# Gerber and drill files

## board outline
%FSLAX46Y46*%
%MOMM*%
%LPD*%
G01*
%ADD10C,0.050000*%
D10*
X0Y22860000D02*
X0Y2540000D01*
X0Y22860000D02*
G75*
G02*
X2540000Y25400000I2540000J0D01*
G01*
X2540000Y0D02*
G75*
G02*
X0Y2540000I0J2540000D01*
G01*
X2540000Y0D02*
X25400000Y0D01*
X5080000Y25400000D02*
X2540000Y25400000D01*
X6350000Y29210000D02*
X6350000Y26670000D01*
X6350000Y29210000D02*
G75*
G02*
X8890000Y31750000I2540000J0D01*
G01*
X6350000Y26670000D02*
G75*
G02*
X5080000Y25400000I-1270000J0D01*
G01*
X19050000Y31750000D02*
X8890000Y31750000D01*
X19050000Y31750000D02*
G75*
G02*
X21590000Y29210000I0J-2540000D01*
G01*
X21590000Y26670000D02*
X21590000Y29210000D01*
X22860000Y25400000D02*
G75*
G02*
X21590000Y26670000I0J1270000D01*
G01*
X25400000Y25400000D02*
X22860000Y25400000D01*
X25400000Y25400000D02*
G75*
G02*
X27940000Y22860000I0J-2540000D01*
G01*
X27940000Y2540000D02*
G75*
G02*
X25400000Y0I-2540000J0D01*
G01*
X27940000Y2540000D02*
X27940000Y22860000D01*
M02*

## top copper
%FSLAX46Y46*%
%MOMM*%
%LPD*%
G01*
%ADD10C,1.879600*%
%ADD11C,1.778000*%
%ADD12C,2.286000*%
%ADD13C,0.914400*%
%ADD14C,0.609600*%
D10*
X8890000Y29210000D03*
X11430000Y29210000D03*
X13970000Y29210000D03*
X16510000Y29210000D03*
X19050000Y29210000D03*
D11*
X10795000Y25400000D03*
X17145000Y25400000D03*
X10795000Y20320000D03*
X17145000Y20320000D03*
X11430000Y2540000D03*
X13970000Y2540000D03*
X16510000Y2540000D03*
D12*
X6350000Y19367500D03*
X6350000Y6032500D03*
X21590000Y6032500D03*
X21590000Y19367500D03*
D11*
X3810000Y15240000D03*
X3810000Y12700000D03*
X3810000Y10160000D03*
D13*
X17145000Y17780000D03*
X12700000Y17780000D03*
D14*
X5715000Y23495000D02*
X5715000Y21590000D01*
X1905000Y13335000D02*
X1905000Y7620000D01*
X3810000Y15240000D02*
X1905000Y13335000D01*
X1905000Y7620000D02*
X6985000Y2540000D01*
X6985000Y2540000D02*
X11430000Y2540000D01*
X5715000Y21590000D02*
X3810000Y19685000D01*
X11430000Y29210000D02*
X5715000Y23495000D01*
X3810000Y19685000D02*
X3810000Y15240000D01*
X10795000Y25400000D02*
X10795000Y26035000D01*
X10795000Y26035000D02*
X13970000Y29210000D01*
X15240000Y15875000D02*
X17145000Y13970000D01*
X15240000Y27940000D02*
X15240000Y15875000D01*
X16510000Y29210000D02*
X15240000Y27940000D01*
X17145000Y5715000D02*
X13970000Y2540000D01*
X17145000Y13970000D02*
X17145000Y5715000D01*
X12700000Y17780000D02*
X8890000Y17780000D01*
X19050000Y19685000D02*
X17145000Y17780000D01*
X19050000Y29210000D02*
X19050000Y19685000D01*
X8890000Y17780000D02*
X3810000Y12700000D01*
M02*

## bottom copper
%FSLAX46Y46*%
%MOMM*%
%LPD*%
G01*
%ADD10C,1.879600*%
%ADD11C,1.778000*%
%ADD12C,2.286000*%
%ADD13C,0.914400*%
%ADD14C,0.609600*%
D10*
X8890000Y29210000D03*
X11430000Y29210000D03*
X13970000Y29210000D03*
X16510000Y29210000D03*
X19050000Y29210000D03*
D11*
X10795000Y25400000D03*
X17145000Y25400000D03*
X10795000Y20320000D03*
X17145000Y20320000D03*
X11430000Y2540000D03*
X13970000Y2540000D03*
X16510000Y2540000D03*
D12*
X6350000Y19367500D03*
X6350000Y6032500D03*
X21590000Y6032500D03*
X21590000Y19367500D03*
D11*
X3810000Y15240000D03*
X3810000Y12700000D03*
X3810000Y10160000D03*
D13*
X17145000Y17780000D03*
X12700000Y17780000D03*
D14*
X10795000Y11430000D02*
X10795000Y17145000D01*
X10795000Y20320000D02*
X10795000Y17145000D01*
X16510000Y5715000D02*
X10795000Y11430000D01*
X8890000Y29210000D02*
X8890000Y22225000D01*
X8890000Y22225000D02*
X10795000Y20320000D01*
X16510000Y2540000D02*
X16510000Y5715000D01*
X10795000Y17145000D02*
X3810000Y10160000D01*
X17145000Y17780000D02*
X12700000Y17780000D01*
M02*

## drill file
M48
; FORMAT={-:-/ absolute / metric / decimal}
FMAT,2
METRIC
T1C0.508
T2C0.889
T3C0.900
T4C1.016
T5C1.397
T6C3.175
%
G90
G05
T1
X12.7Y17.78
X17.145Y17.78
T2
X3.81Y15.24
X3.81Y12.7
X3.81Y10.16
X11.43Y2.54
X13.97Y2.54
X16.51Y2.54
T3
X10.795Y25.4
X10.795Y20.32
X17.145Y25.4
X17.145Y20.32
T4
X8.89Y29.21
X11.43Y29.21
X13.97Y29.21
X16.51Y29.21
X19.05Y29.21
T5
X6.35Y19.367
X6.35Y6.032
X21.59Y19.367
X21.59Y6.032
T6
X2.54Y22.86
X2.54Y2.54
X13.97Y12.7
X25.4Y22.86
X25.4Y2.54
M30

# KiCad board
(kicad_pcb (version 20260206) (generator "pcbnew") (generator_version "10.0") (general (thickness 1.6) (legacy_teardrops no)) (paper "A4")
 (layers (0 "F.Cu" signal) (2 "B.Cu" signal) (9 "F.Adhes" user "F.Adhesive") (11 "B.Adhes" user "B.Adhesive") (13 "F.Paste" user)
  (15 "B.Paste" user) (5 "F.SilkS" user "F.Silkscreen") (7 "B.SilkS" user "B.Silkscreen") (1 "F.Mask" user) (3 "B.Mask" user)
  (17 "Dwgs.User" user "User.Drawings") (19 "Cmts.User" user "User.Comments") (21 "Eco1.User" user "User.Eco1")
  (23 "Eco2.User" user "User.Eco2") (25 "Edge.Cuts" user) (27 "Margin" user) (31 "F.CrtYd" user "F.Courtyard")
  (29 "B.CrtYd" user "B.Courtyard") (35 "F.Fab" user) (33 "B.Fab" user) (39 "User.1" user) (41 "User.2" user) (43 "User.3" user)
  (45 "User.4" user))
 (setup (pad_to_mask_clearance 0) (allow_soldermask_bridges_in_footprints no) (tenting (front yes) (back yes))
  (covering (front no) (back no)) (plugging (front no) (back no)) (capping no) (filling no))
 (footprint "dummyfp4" (layer "F.Cu") (at 13.97 -12.7)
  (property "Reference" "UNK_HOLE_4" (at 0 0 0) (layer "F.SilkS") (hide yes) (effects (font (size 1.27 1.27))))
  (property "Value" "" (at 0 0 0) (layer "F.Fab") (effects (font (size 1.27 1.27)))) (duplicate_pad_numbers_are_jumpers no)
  (pad "" np_thru_hole circle (at 0 0) (size 3.175 3.175) (drill 3.175) (layers "*.Cu" "*.Mask")))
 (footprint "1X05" (layer "F.Cu") (at 8.89 -29.21)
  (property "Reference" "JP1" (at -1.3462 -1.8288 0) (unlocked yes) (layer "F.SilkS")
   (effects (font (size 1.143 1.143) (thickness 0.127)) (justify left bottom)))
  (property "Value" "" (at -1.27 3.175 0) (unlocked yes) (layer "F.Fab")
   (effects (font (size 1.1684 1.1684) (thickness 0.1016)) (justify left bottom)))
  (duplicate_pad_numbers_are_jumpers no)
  (pad "1" thru_hole circle (at 0 0 90) (size 1.8796 1.8796) (drill 1.016) (layers "*.Cu" "*.Mask") (remove_unused_layers no) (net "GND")
   (solder_mask_margin 0.1016) (thermal_bridge_angle 0))
  (pad "2" thru_hole circle (at 2.54 0 90) (size 1.8796 1.8796) (drill 1.016) (layers "*.Cu" "*.Mask") (remove_unused_layers no) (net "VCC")
   (solder_mask_margin 0.1016) (thermal_bridge_angle 0))
  (pad "3" thru_hole circle (at 5.08 0 90) (size 1.8796 1.8796) (drill 1.016) (layers "*.Cu" "*.Mask") (remove_unused_layers no) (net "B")
   (solder_mask_margin 0.1016) (thermal_bridge_angle 0))
  (pad "4" thru_hole circle (at 7.62 0 90) (size 1.8796 1.8796) (drill 1.016) (layers "*.Cu" "*.Mask") (remove_unused_layers no) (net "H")
   (solder_mask_margin 0.1016) (thermal_bridge_angle 0))
  (pad "5" thru_hole circle (at 10.16 0 90) (size 1.8796 1.8796) (drill 1.016) (layers "*.Cu" "*.Mask") (remove_unused_layers no) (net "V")
   (solder_mask_margin 0.1016) (thermal_bridge_angle 0)))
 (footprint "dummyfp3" (layer "F.Cu") (at 25.4 -22.86)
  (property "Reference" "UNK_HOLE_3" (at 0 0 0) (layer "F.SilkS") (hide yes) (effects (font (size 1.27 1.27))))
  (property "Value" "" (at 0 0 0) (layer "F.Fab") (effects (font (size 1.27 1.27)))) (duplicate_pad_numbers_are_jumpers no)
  (pad "" np_thru_hole circle (at 0 0) (size 3.175 3.175) (drill 3.175) (layers "*.Cu" "*.Mask")))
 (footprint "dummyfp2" (layer "F.Cu") (at 2.54 -22.86)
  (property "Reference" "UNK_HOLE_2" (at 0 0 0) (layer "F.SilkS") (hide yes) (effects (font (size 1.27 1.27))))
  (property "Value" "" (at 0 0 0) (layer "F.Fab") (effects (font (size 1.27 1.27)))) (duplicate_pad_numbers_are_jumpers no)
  (pad "" np_thru_hole circle (at 0 0) (size 3.175 3.175) (drill 3.175) (layers "*.Cu" "*.Mask")))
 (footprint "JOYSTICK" (layer "F.Cu") (at 13.97 -12.7)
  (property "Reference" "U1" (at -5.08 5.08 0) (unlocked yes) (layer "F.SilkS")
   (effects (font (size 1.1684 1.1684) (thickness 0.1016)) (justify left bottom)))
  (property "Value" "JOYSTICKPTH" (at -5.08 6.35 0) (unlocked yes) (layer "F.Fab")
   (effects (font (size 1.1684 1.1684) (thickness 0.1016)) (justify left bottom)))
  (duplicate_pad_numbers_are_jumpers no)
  (pad "B1A" thru_hole circle (at -3.175 -12.7) (size 1.778 1.778) (drill 0.9) (layers "*.Cu" "*.Mask") (remove_unused_layers no) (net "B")
   (solder_mask_margin 0.1016) (thermal_bridge_angle 0))
  (pad "B1B" thru_hole circle (at 3.175 -12.7) (size 1.778 1.778) (drill 0.9) (layers "*.Cu" "*.Mask") (remove_unused_layers no)
   (solder_mask_margin 0.1016) (thermal_bridge_angle 0))
  (pad "B2A" thru_hole circle (at -3.175 -7.62) (size 1.778 1.778) (drill 0.9) (layers "*.Cu" "*.Mask") (remove_unused_layers no)
   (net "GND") (solder_mask_margin 0.1016) (thermal_bridge_angle 0))
  (pad "B2B" thru_hole circle (at 3.175 -7.62) (size 1.778 1.778) (drill 0.9) (layers "*.Cu" "*.Mask") (remove_unused_layers no)
   (solder_mask_margin 0.1016) (thermal_bridge_angle 0))
  (pad "H1" thru_hole circle (at -2.54 10.16) (size 1.778 1.778) (drill 0.889) (layers "*.Cu" "*.Mask") (remove_unused_layers no)
   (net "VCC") (solder_mask_margin 0.1016) (thermal_bridge_angle 0))
  (pad "H2" thru_hole circle (at 0 10.16) (size 1.778 1.778) (drill 0.889) (layers "*.Cu" "*.Mask") (remove_unused_layers no) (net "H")
   (solder_mask_margin 0.1016) (thermal_bridge_angle 0))
  (pad "H3" thru_hole circle (at 2.54 10.16) (size 1.778 1.778) (drill 0.889) (layers "*.Cu" "*.Mask") (remove_unused_layers no) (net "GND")
   (solder_mask_margin 0.1016) (thermal_bridge_angle 0))
  (pad "MOUNT1" thru_hole circle (at -7.62 -6.6675) (size 2.286 2.286) (drill 1.397) (layers "*.Cu" "*.Mask") (remove_unused_layers no)
   (solder_mask_margin 0.1016) (thermal_bridge_angle 0))
  (pad "MOUNT2" thru_hole circle (at -7.62 6.6675) (size 2.286 2.286) (drill 1.397) (layers "*.Cu" "*.Mask") (remove_unused_layers no)
   (solder_mask_margin 0.1016) (thermal_bridge_angle 0))
  (pad "MOUNT3" thru_hole circle (at 7.62 6.6675) (size 2.286 2.286) (drill 1.397) (layers "*.Cu" "*.Mask") (remove_unused_layers no)
   (solder_mask_margin 0.1016) (thermal_bridge_angle 0))
  (pad "MOUNT4" thru_hole circle (at 7.62 -6.6675) (size 2.286 2.286) (drill 1.397) (layers "*.Cu" "*.Mask") (remove_unused_layers no)
   (solder_mask_margin 0.1016) (thermal_bridge_angle 0))
  (pad "V1" thru_hole circle (at -10.16 -2.54) (size 1.778 1.778) (drill 0.889) (layers "*.Cu" "*.Mask") (remove_unused_layers no)
   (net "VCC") (solder_mask_margin 0.1016) (thermal_bridge_angle 0))
  (pad "V2" thru_hole circle (at -10.16 0) (size 1.778 1.778) (drill 0.889) (layers "*.Cu" "*.Mask") (remove_unused_layers no) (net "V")
   (solder_mask_margin 0.1016) (thermal_bridge_angle 0))
  (pad "V3" thru_hole circle (at -10.16 2.54) (size 1.778 1.778) (drill 0.889) (layers "*.Cu" "*.Mask") (remove_unused_layers no)
   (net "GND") (solder_mask_margin 0.1016) (thermal_bridge_angle 0)))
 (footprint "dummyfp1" (layer "F.Cu") (at 25.4 -2.54)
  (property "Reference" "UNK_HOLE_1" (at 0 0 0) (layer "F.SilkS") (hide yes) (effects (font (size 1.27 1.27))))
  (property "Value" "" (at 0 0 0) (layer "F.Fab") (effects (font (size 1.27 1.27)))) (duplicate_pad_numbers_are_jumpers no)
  (pad "" np_thru_hole circle (at 0 0) (size 3.175 3.175) (drill 3.175) (layers "*.Cu" "*.Mask")))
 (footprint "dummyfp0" (layer "F.Cu") (at 2.54 -2.54)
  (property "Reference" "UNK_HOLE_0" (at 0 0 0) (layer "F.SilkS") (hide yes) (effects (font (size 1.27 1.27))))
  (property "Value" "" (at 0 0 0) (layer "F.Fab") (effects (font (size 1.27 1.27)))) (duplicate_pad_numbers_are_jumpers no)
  (pad "" np_thru_hole circle (at 0 0) (size 3.175 3.175) (drill 3.175) (layers "*.Cu" "*.Mask")))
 (gr_line (start 0 -22.86) (end 0 -2.54) (stroke (width 0.05) (type solid)) (layer "Edge.Cuts"))
 (gr_arc (start 0 -22.86) (mid 0.743949 -24.656051) (end 2.54 -25.4) (stroke (width 0.05) (type solid)) (layer "Edge.Cuts"))
 (gr_arc (start 2.54 0) (mid 0.743949 -0.743949) (end 0 -2.54) (stroke (width 0.05) (type solid)) (layer "Edge.Cuts"))
 (gr_line (start 2.54 0) (end 25.4 0) (stroke (width 0.05) (type solid)) (layer "Edge.Cuts"))
 (gr_line (start 5.08 -25.4) (end 2.54 -25.4) (stroke (width 0.05) (type solid)) (layer "Edge.Cuts"))
 (gr_line (start 6.35 -29.21) (end 6.35 -26.67) (stroke (width 0.05) (type solid)) (layer "Edge.Cuts"))
 (gr_arc (start 6.35 -29.21) (mid 7.093949 -31.006051) (end 8.89 -31.75) (stroke (width 0.05) (type solid)) (layer "Edge.Cuts"))
 (gr_arc (start 6.35 -26.67) (mid 5.978026 -25.771974) (end 5.08 -25.4) (stroke (width 0.05) (type solid)) (layer "Edge.Cuts"))
 (gr_line (start 19.05 -31.75) (end 8.89 -31.75) (stroke (width 0.05) (type solid)) (layer "Edge.Cuts"))
 (gr_arc (start 19.05 -31.75) (mid 20.846051 -31.006051) (end 21.59 -29.21) (stroke (width 0.05) (type solid)) (layer "Edge.Cuts"))
 (gr_line (start 21.59 -26.67) (end 21.59 -29.21) (stroke (width 0.05) (type solid)) (layer "Edge.Cuts"))
 (gr_arc (start 22.86 -25.4) (mid 21.961974 -25.771974) (end 21.59 -26.67) (stroke (width 0.05) (type solid)) (layer "Edge.Cuts"))
 (gr_line (start 25.4 -25.4) (end 22.86 -25.4) (stroke (width 0.05) (type solid)) (layer "Edge.Cuts"))
 (gr_arc (start 25.4 -25.4) (mid 27.196051 -24.656051) (end 27.94 -22.86) (stroke (width 0.05) (type solid)) (layer "Edge.Cuts"))
 (gr_arc (start 27.94 -2.54) (mid 27.196051 -0.743949) (end 25.4 0) (stroke (width 0.05) (type solid)) (layer "Edge.Cuts"))
 (gr_line (start 27.94 -2.54) (end 27.94 -22.86) (stroke (width 0.05) (type solid)) (layer "Edge.Cuts"))
 (segment (start 10.795 -11.43) (end 10.795 -17.145) (width 0.6096) (layer "B.Cu") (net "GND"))
 (segment (start 10.795 -20.32) (end 10.795 -17.145) (width 0.6096) (layer "B.Cu") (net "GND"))
 (segment (start 16.51 -5.715) (end 10.795 -11.43) (width 0.6096) (layer "B.Cu") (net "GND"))
 (segment (start 8.89 -29.21) (end 8.89 -22.225) (width 0.6096) (layer "B.Cu") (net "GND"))
 (segment (start 8.89 -22.225) (end 10.795 -20.32) (width 0.6096) (layer "B.Cu") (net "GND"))
 (segment (start 16.51 -2.54) (end 16.51 -5.715) (width 0.6096) (layer "B.Cu") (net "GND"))
 (segment (start 10.795 -17.145) (end 3.81 -10.16) (width 0.6096) (layer "B.Cu") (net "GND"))
 (segment (start 5.715 -23.495) (end 5.715 -21.59) (width 0.6096) (layer "F.Cu") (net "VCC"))
 (segment (start 1.905 -13.335) (end 1.905 -7.62) (width 0.6096) (layer "F.Cu") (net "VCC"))
 (segment (start 3.81 -15.24) (end 1.905 -13.335) (width 0.6096) (layer "F.Cu") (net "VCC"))
 (segment (start 1.905 -7.62) (end 6.985 -2.54) (width 0.6096) (layer "F.Cu") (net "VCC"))
 (segment (start 6.985 -2.54) (end 11.43 -2.54) (width 0.6096) (layer "F.Cu") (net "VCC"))
 (segment (start 5.715 -21.59) (end 3.81 -19.685) (width 0.6096) (layer "F.Cu") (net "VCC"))
 (segment (start 11.43 -29.21) (end 5.715 -23.495) (width 0.6096) (layer "F.Cu") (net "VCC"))
 (segment (start 3.81 -19.685) (end 3.81 -15.24) (width 0.6096) (layer "F.Cu") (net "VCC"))
 (segment (start 10.795 -25.4) (end 10.795 -26.035) (width 0.6096) (layer "F.Cu") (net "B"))
 (segment (start 10.795 -26.035) (end 13.97 -29.21) (width 0.6096) (layer "F.Cu") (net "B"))
 (segment (start 15.24 -15.875) (end 17.145 -13.97) (width 0.6096) (layer "F.Cu") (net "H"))
 (segment (start 15.24 -27.94) (end 15.24 -15.875) (width 0.6096) (layer "F.Cu") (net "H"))
 (segment (start 16.51 -29.21) (end 15.24 -27.94) (width 0.6096) (layer "F.Cu") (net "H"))
 (segment (start 17.145 -5.715) (end 13.97 -2.54) (width 0.6096) (layer "F.Cu") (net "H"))
 (segment (start 17.145 -13.97) (end 17.145 -5.715) (width 0.6096) (layer "F.Cu") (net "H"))
 (segment (start 12.7 -17.78) (end 8.89 -17.78) (width 0.6096) (layer "F.Cu") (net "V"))
 (segment (start 19.05 -19.685) (end 17.145 -17.78) (width 0.6096) (layer "F.Cu") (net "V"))
 (segment (start 19.05 -29.21) (end 19.05 -19.685) (width 0.6096) (layer "F.Cu") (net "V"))
 (segment (start 8.89 -17.78) (end 3.81 -12.7) (width 0.6096) (layer "F.Cu") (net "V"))
 (via (at 17.145 -17.78) (size 0.9144) (drill 0.508) (layers "F.Cu" "B.Cu") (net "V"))
 (via (at 12.7 -17.78) (size 0.9144) (drill 0.508) (layers "F.Cu" "B.Cu") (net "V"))
 (segment (start 17.145 -17.78) (end 12.7 -17.78) (width 0.6096) (layer "B.Cu") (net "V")))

